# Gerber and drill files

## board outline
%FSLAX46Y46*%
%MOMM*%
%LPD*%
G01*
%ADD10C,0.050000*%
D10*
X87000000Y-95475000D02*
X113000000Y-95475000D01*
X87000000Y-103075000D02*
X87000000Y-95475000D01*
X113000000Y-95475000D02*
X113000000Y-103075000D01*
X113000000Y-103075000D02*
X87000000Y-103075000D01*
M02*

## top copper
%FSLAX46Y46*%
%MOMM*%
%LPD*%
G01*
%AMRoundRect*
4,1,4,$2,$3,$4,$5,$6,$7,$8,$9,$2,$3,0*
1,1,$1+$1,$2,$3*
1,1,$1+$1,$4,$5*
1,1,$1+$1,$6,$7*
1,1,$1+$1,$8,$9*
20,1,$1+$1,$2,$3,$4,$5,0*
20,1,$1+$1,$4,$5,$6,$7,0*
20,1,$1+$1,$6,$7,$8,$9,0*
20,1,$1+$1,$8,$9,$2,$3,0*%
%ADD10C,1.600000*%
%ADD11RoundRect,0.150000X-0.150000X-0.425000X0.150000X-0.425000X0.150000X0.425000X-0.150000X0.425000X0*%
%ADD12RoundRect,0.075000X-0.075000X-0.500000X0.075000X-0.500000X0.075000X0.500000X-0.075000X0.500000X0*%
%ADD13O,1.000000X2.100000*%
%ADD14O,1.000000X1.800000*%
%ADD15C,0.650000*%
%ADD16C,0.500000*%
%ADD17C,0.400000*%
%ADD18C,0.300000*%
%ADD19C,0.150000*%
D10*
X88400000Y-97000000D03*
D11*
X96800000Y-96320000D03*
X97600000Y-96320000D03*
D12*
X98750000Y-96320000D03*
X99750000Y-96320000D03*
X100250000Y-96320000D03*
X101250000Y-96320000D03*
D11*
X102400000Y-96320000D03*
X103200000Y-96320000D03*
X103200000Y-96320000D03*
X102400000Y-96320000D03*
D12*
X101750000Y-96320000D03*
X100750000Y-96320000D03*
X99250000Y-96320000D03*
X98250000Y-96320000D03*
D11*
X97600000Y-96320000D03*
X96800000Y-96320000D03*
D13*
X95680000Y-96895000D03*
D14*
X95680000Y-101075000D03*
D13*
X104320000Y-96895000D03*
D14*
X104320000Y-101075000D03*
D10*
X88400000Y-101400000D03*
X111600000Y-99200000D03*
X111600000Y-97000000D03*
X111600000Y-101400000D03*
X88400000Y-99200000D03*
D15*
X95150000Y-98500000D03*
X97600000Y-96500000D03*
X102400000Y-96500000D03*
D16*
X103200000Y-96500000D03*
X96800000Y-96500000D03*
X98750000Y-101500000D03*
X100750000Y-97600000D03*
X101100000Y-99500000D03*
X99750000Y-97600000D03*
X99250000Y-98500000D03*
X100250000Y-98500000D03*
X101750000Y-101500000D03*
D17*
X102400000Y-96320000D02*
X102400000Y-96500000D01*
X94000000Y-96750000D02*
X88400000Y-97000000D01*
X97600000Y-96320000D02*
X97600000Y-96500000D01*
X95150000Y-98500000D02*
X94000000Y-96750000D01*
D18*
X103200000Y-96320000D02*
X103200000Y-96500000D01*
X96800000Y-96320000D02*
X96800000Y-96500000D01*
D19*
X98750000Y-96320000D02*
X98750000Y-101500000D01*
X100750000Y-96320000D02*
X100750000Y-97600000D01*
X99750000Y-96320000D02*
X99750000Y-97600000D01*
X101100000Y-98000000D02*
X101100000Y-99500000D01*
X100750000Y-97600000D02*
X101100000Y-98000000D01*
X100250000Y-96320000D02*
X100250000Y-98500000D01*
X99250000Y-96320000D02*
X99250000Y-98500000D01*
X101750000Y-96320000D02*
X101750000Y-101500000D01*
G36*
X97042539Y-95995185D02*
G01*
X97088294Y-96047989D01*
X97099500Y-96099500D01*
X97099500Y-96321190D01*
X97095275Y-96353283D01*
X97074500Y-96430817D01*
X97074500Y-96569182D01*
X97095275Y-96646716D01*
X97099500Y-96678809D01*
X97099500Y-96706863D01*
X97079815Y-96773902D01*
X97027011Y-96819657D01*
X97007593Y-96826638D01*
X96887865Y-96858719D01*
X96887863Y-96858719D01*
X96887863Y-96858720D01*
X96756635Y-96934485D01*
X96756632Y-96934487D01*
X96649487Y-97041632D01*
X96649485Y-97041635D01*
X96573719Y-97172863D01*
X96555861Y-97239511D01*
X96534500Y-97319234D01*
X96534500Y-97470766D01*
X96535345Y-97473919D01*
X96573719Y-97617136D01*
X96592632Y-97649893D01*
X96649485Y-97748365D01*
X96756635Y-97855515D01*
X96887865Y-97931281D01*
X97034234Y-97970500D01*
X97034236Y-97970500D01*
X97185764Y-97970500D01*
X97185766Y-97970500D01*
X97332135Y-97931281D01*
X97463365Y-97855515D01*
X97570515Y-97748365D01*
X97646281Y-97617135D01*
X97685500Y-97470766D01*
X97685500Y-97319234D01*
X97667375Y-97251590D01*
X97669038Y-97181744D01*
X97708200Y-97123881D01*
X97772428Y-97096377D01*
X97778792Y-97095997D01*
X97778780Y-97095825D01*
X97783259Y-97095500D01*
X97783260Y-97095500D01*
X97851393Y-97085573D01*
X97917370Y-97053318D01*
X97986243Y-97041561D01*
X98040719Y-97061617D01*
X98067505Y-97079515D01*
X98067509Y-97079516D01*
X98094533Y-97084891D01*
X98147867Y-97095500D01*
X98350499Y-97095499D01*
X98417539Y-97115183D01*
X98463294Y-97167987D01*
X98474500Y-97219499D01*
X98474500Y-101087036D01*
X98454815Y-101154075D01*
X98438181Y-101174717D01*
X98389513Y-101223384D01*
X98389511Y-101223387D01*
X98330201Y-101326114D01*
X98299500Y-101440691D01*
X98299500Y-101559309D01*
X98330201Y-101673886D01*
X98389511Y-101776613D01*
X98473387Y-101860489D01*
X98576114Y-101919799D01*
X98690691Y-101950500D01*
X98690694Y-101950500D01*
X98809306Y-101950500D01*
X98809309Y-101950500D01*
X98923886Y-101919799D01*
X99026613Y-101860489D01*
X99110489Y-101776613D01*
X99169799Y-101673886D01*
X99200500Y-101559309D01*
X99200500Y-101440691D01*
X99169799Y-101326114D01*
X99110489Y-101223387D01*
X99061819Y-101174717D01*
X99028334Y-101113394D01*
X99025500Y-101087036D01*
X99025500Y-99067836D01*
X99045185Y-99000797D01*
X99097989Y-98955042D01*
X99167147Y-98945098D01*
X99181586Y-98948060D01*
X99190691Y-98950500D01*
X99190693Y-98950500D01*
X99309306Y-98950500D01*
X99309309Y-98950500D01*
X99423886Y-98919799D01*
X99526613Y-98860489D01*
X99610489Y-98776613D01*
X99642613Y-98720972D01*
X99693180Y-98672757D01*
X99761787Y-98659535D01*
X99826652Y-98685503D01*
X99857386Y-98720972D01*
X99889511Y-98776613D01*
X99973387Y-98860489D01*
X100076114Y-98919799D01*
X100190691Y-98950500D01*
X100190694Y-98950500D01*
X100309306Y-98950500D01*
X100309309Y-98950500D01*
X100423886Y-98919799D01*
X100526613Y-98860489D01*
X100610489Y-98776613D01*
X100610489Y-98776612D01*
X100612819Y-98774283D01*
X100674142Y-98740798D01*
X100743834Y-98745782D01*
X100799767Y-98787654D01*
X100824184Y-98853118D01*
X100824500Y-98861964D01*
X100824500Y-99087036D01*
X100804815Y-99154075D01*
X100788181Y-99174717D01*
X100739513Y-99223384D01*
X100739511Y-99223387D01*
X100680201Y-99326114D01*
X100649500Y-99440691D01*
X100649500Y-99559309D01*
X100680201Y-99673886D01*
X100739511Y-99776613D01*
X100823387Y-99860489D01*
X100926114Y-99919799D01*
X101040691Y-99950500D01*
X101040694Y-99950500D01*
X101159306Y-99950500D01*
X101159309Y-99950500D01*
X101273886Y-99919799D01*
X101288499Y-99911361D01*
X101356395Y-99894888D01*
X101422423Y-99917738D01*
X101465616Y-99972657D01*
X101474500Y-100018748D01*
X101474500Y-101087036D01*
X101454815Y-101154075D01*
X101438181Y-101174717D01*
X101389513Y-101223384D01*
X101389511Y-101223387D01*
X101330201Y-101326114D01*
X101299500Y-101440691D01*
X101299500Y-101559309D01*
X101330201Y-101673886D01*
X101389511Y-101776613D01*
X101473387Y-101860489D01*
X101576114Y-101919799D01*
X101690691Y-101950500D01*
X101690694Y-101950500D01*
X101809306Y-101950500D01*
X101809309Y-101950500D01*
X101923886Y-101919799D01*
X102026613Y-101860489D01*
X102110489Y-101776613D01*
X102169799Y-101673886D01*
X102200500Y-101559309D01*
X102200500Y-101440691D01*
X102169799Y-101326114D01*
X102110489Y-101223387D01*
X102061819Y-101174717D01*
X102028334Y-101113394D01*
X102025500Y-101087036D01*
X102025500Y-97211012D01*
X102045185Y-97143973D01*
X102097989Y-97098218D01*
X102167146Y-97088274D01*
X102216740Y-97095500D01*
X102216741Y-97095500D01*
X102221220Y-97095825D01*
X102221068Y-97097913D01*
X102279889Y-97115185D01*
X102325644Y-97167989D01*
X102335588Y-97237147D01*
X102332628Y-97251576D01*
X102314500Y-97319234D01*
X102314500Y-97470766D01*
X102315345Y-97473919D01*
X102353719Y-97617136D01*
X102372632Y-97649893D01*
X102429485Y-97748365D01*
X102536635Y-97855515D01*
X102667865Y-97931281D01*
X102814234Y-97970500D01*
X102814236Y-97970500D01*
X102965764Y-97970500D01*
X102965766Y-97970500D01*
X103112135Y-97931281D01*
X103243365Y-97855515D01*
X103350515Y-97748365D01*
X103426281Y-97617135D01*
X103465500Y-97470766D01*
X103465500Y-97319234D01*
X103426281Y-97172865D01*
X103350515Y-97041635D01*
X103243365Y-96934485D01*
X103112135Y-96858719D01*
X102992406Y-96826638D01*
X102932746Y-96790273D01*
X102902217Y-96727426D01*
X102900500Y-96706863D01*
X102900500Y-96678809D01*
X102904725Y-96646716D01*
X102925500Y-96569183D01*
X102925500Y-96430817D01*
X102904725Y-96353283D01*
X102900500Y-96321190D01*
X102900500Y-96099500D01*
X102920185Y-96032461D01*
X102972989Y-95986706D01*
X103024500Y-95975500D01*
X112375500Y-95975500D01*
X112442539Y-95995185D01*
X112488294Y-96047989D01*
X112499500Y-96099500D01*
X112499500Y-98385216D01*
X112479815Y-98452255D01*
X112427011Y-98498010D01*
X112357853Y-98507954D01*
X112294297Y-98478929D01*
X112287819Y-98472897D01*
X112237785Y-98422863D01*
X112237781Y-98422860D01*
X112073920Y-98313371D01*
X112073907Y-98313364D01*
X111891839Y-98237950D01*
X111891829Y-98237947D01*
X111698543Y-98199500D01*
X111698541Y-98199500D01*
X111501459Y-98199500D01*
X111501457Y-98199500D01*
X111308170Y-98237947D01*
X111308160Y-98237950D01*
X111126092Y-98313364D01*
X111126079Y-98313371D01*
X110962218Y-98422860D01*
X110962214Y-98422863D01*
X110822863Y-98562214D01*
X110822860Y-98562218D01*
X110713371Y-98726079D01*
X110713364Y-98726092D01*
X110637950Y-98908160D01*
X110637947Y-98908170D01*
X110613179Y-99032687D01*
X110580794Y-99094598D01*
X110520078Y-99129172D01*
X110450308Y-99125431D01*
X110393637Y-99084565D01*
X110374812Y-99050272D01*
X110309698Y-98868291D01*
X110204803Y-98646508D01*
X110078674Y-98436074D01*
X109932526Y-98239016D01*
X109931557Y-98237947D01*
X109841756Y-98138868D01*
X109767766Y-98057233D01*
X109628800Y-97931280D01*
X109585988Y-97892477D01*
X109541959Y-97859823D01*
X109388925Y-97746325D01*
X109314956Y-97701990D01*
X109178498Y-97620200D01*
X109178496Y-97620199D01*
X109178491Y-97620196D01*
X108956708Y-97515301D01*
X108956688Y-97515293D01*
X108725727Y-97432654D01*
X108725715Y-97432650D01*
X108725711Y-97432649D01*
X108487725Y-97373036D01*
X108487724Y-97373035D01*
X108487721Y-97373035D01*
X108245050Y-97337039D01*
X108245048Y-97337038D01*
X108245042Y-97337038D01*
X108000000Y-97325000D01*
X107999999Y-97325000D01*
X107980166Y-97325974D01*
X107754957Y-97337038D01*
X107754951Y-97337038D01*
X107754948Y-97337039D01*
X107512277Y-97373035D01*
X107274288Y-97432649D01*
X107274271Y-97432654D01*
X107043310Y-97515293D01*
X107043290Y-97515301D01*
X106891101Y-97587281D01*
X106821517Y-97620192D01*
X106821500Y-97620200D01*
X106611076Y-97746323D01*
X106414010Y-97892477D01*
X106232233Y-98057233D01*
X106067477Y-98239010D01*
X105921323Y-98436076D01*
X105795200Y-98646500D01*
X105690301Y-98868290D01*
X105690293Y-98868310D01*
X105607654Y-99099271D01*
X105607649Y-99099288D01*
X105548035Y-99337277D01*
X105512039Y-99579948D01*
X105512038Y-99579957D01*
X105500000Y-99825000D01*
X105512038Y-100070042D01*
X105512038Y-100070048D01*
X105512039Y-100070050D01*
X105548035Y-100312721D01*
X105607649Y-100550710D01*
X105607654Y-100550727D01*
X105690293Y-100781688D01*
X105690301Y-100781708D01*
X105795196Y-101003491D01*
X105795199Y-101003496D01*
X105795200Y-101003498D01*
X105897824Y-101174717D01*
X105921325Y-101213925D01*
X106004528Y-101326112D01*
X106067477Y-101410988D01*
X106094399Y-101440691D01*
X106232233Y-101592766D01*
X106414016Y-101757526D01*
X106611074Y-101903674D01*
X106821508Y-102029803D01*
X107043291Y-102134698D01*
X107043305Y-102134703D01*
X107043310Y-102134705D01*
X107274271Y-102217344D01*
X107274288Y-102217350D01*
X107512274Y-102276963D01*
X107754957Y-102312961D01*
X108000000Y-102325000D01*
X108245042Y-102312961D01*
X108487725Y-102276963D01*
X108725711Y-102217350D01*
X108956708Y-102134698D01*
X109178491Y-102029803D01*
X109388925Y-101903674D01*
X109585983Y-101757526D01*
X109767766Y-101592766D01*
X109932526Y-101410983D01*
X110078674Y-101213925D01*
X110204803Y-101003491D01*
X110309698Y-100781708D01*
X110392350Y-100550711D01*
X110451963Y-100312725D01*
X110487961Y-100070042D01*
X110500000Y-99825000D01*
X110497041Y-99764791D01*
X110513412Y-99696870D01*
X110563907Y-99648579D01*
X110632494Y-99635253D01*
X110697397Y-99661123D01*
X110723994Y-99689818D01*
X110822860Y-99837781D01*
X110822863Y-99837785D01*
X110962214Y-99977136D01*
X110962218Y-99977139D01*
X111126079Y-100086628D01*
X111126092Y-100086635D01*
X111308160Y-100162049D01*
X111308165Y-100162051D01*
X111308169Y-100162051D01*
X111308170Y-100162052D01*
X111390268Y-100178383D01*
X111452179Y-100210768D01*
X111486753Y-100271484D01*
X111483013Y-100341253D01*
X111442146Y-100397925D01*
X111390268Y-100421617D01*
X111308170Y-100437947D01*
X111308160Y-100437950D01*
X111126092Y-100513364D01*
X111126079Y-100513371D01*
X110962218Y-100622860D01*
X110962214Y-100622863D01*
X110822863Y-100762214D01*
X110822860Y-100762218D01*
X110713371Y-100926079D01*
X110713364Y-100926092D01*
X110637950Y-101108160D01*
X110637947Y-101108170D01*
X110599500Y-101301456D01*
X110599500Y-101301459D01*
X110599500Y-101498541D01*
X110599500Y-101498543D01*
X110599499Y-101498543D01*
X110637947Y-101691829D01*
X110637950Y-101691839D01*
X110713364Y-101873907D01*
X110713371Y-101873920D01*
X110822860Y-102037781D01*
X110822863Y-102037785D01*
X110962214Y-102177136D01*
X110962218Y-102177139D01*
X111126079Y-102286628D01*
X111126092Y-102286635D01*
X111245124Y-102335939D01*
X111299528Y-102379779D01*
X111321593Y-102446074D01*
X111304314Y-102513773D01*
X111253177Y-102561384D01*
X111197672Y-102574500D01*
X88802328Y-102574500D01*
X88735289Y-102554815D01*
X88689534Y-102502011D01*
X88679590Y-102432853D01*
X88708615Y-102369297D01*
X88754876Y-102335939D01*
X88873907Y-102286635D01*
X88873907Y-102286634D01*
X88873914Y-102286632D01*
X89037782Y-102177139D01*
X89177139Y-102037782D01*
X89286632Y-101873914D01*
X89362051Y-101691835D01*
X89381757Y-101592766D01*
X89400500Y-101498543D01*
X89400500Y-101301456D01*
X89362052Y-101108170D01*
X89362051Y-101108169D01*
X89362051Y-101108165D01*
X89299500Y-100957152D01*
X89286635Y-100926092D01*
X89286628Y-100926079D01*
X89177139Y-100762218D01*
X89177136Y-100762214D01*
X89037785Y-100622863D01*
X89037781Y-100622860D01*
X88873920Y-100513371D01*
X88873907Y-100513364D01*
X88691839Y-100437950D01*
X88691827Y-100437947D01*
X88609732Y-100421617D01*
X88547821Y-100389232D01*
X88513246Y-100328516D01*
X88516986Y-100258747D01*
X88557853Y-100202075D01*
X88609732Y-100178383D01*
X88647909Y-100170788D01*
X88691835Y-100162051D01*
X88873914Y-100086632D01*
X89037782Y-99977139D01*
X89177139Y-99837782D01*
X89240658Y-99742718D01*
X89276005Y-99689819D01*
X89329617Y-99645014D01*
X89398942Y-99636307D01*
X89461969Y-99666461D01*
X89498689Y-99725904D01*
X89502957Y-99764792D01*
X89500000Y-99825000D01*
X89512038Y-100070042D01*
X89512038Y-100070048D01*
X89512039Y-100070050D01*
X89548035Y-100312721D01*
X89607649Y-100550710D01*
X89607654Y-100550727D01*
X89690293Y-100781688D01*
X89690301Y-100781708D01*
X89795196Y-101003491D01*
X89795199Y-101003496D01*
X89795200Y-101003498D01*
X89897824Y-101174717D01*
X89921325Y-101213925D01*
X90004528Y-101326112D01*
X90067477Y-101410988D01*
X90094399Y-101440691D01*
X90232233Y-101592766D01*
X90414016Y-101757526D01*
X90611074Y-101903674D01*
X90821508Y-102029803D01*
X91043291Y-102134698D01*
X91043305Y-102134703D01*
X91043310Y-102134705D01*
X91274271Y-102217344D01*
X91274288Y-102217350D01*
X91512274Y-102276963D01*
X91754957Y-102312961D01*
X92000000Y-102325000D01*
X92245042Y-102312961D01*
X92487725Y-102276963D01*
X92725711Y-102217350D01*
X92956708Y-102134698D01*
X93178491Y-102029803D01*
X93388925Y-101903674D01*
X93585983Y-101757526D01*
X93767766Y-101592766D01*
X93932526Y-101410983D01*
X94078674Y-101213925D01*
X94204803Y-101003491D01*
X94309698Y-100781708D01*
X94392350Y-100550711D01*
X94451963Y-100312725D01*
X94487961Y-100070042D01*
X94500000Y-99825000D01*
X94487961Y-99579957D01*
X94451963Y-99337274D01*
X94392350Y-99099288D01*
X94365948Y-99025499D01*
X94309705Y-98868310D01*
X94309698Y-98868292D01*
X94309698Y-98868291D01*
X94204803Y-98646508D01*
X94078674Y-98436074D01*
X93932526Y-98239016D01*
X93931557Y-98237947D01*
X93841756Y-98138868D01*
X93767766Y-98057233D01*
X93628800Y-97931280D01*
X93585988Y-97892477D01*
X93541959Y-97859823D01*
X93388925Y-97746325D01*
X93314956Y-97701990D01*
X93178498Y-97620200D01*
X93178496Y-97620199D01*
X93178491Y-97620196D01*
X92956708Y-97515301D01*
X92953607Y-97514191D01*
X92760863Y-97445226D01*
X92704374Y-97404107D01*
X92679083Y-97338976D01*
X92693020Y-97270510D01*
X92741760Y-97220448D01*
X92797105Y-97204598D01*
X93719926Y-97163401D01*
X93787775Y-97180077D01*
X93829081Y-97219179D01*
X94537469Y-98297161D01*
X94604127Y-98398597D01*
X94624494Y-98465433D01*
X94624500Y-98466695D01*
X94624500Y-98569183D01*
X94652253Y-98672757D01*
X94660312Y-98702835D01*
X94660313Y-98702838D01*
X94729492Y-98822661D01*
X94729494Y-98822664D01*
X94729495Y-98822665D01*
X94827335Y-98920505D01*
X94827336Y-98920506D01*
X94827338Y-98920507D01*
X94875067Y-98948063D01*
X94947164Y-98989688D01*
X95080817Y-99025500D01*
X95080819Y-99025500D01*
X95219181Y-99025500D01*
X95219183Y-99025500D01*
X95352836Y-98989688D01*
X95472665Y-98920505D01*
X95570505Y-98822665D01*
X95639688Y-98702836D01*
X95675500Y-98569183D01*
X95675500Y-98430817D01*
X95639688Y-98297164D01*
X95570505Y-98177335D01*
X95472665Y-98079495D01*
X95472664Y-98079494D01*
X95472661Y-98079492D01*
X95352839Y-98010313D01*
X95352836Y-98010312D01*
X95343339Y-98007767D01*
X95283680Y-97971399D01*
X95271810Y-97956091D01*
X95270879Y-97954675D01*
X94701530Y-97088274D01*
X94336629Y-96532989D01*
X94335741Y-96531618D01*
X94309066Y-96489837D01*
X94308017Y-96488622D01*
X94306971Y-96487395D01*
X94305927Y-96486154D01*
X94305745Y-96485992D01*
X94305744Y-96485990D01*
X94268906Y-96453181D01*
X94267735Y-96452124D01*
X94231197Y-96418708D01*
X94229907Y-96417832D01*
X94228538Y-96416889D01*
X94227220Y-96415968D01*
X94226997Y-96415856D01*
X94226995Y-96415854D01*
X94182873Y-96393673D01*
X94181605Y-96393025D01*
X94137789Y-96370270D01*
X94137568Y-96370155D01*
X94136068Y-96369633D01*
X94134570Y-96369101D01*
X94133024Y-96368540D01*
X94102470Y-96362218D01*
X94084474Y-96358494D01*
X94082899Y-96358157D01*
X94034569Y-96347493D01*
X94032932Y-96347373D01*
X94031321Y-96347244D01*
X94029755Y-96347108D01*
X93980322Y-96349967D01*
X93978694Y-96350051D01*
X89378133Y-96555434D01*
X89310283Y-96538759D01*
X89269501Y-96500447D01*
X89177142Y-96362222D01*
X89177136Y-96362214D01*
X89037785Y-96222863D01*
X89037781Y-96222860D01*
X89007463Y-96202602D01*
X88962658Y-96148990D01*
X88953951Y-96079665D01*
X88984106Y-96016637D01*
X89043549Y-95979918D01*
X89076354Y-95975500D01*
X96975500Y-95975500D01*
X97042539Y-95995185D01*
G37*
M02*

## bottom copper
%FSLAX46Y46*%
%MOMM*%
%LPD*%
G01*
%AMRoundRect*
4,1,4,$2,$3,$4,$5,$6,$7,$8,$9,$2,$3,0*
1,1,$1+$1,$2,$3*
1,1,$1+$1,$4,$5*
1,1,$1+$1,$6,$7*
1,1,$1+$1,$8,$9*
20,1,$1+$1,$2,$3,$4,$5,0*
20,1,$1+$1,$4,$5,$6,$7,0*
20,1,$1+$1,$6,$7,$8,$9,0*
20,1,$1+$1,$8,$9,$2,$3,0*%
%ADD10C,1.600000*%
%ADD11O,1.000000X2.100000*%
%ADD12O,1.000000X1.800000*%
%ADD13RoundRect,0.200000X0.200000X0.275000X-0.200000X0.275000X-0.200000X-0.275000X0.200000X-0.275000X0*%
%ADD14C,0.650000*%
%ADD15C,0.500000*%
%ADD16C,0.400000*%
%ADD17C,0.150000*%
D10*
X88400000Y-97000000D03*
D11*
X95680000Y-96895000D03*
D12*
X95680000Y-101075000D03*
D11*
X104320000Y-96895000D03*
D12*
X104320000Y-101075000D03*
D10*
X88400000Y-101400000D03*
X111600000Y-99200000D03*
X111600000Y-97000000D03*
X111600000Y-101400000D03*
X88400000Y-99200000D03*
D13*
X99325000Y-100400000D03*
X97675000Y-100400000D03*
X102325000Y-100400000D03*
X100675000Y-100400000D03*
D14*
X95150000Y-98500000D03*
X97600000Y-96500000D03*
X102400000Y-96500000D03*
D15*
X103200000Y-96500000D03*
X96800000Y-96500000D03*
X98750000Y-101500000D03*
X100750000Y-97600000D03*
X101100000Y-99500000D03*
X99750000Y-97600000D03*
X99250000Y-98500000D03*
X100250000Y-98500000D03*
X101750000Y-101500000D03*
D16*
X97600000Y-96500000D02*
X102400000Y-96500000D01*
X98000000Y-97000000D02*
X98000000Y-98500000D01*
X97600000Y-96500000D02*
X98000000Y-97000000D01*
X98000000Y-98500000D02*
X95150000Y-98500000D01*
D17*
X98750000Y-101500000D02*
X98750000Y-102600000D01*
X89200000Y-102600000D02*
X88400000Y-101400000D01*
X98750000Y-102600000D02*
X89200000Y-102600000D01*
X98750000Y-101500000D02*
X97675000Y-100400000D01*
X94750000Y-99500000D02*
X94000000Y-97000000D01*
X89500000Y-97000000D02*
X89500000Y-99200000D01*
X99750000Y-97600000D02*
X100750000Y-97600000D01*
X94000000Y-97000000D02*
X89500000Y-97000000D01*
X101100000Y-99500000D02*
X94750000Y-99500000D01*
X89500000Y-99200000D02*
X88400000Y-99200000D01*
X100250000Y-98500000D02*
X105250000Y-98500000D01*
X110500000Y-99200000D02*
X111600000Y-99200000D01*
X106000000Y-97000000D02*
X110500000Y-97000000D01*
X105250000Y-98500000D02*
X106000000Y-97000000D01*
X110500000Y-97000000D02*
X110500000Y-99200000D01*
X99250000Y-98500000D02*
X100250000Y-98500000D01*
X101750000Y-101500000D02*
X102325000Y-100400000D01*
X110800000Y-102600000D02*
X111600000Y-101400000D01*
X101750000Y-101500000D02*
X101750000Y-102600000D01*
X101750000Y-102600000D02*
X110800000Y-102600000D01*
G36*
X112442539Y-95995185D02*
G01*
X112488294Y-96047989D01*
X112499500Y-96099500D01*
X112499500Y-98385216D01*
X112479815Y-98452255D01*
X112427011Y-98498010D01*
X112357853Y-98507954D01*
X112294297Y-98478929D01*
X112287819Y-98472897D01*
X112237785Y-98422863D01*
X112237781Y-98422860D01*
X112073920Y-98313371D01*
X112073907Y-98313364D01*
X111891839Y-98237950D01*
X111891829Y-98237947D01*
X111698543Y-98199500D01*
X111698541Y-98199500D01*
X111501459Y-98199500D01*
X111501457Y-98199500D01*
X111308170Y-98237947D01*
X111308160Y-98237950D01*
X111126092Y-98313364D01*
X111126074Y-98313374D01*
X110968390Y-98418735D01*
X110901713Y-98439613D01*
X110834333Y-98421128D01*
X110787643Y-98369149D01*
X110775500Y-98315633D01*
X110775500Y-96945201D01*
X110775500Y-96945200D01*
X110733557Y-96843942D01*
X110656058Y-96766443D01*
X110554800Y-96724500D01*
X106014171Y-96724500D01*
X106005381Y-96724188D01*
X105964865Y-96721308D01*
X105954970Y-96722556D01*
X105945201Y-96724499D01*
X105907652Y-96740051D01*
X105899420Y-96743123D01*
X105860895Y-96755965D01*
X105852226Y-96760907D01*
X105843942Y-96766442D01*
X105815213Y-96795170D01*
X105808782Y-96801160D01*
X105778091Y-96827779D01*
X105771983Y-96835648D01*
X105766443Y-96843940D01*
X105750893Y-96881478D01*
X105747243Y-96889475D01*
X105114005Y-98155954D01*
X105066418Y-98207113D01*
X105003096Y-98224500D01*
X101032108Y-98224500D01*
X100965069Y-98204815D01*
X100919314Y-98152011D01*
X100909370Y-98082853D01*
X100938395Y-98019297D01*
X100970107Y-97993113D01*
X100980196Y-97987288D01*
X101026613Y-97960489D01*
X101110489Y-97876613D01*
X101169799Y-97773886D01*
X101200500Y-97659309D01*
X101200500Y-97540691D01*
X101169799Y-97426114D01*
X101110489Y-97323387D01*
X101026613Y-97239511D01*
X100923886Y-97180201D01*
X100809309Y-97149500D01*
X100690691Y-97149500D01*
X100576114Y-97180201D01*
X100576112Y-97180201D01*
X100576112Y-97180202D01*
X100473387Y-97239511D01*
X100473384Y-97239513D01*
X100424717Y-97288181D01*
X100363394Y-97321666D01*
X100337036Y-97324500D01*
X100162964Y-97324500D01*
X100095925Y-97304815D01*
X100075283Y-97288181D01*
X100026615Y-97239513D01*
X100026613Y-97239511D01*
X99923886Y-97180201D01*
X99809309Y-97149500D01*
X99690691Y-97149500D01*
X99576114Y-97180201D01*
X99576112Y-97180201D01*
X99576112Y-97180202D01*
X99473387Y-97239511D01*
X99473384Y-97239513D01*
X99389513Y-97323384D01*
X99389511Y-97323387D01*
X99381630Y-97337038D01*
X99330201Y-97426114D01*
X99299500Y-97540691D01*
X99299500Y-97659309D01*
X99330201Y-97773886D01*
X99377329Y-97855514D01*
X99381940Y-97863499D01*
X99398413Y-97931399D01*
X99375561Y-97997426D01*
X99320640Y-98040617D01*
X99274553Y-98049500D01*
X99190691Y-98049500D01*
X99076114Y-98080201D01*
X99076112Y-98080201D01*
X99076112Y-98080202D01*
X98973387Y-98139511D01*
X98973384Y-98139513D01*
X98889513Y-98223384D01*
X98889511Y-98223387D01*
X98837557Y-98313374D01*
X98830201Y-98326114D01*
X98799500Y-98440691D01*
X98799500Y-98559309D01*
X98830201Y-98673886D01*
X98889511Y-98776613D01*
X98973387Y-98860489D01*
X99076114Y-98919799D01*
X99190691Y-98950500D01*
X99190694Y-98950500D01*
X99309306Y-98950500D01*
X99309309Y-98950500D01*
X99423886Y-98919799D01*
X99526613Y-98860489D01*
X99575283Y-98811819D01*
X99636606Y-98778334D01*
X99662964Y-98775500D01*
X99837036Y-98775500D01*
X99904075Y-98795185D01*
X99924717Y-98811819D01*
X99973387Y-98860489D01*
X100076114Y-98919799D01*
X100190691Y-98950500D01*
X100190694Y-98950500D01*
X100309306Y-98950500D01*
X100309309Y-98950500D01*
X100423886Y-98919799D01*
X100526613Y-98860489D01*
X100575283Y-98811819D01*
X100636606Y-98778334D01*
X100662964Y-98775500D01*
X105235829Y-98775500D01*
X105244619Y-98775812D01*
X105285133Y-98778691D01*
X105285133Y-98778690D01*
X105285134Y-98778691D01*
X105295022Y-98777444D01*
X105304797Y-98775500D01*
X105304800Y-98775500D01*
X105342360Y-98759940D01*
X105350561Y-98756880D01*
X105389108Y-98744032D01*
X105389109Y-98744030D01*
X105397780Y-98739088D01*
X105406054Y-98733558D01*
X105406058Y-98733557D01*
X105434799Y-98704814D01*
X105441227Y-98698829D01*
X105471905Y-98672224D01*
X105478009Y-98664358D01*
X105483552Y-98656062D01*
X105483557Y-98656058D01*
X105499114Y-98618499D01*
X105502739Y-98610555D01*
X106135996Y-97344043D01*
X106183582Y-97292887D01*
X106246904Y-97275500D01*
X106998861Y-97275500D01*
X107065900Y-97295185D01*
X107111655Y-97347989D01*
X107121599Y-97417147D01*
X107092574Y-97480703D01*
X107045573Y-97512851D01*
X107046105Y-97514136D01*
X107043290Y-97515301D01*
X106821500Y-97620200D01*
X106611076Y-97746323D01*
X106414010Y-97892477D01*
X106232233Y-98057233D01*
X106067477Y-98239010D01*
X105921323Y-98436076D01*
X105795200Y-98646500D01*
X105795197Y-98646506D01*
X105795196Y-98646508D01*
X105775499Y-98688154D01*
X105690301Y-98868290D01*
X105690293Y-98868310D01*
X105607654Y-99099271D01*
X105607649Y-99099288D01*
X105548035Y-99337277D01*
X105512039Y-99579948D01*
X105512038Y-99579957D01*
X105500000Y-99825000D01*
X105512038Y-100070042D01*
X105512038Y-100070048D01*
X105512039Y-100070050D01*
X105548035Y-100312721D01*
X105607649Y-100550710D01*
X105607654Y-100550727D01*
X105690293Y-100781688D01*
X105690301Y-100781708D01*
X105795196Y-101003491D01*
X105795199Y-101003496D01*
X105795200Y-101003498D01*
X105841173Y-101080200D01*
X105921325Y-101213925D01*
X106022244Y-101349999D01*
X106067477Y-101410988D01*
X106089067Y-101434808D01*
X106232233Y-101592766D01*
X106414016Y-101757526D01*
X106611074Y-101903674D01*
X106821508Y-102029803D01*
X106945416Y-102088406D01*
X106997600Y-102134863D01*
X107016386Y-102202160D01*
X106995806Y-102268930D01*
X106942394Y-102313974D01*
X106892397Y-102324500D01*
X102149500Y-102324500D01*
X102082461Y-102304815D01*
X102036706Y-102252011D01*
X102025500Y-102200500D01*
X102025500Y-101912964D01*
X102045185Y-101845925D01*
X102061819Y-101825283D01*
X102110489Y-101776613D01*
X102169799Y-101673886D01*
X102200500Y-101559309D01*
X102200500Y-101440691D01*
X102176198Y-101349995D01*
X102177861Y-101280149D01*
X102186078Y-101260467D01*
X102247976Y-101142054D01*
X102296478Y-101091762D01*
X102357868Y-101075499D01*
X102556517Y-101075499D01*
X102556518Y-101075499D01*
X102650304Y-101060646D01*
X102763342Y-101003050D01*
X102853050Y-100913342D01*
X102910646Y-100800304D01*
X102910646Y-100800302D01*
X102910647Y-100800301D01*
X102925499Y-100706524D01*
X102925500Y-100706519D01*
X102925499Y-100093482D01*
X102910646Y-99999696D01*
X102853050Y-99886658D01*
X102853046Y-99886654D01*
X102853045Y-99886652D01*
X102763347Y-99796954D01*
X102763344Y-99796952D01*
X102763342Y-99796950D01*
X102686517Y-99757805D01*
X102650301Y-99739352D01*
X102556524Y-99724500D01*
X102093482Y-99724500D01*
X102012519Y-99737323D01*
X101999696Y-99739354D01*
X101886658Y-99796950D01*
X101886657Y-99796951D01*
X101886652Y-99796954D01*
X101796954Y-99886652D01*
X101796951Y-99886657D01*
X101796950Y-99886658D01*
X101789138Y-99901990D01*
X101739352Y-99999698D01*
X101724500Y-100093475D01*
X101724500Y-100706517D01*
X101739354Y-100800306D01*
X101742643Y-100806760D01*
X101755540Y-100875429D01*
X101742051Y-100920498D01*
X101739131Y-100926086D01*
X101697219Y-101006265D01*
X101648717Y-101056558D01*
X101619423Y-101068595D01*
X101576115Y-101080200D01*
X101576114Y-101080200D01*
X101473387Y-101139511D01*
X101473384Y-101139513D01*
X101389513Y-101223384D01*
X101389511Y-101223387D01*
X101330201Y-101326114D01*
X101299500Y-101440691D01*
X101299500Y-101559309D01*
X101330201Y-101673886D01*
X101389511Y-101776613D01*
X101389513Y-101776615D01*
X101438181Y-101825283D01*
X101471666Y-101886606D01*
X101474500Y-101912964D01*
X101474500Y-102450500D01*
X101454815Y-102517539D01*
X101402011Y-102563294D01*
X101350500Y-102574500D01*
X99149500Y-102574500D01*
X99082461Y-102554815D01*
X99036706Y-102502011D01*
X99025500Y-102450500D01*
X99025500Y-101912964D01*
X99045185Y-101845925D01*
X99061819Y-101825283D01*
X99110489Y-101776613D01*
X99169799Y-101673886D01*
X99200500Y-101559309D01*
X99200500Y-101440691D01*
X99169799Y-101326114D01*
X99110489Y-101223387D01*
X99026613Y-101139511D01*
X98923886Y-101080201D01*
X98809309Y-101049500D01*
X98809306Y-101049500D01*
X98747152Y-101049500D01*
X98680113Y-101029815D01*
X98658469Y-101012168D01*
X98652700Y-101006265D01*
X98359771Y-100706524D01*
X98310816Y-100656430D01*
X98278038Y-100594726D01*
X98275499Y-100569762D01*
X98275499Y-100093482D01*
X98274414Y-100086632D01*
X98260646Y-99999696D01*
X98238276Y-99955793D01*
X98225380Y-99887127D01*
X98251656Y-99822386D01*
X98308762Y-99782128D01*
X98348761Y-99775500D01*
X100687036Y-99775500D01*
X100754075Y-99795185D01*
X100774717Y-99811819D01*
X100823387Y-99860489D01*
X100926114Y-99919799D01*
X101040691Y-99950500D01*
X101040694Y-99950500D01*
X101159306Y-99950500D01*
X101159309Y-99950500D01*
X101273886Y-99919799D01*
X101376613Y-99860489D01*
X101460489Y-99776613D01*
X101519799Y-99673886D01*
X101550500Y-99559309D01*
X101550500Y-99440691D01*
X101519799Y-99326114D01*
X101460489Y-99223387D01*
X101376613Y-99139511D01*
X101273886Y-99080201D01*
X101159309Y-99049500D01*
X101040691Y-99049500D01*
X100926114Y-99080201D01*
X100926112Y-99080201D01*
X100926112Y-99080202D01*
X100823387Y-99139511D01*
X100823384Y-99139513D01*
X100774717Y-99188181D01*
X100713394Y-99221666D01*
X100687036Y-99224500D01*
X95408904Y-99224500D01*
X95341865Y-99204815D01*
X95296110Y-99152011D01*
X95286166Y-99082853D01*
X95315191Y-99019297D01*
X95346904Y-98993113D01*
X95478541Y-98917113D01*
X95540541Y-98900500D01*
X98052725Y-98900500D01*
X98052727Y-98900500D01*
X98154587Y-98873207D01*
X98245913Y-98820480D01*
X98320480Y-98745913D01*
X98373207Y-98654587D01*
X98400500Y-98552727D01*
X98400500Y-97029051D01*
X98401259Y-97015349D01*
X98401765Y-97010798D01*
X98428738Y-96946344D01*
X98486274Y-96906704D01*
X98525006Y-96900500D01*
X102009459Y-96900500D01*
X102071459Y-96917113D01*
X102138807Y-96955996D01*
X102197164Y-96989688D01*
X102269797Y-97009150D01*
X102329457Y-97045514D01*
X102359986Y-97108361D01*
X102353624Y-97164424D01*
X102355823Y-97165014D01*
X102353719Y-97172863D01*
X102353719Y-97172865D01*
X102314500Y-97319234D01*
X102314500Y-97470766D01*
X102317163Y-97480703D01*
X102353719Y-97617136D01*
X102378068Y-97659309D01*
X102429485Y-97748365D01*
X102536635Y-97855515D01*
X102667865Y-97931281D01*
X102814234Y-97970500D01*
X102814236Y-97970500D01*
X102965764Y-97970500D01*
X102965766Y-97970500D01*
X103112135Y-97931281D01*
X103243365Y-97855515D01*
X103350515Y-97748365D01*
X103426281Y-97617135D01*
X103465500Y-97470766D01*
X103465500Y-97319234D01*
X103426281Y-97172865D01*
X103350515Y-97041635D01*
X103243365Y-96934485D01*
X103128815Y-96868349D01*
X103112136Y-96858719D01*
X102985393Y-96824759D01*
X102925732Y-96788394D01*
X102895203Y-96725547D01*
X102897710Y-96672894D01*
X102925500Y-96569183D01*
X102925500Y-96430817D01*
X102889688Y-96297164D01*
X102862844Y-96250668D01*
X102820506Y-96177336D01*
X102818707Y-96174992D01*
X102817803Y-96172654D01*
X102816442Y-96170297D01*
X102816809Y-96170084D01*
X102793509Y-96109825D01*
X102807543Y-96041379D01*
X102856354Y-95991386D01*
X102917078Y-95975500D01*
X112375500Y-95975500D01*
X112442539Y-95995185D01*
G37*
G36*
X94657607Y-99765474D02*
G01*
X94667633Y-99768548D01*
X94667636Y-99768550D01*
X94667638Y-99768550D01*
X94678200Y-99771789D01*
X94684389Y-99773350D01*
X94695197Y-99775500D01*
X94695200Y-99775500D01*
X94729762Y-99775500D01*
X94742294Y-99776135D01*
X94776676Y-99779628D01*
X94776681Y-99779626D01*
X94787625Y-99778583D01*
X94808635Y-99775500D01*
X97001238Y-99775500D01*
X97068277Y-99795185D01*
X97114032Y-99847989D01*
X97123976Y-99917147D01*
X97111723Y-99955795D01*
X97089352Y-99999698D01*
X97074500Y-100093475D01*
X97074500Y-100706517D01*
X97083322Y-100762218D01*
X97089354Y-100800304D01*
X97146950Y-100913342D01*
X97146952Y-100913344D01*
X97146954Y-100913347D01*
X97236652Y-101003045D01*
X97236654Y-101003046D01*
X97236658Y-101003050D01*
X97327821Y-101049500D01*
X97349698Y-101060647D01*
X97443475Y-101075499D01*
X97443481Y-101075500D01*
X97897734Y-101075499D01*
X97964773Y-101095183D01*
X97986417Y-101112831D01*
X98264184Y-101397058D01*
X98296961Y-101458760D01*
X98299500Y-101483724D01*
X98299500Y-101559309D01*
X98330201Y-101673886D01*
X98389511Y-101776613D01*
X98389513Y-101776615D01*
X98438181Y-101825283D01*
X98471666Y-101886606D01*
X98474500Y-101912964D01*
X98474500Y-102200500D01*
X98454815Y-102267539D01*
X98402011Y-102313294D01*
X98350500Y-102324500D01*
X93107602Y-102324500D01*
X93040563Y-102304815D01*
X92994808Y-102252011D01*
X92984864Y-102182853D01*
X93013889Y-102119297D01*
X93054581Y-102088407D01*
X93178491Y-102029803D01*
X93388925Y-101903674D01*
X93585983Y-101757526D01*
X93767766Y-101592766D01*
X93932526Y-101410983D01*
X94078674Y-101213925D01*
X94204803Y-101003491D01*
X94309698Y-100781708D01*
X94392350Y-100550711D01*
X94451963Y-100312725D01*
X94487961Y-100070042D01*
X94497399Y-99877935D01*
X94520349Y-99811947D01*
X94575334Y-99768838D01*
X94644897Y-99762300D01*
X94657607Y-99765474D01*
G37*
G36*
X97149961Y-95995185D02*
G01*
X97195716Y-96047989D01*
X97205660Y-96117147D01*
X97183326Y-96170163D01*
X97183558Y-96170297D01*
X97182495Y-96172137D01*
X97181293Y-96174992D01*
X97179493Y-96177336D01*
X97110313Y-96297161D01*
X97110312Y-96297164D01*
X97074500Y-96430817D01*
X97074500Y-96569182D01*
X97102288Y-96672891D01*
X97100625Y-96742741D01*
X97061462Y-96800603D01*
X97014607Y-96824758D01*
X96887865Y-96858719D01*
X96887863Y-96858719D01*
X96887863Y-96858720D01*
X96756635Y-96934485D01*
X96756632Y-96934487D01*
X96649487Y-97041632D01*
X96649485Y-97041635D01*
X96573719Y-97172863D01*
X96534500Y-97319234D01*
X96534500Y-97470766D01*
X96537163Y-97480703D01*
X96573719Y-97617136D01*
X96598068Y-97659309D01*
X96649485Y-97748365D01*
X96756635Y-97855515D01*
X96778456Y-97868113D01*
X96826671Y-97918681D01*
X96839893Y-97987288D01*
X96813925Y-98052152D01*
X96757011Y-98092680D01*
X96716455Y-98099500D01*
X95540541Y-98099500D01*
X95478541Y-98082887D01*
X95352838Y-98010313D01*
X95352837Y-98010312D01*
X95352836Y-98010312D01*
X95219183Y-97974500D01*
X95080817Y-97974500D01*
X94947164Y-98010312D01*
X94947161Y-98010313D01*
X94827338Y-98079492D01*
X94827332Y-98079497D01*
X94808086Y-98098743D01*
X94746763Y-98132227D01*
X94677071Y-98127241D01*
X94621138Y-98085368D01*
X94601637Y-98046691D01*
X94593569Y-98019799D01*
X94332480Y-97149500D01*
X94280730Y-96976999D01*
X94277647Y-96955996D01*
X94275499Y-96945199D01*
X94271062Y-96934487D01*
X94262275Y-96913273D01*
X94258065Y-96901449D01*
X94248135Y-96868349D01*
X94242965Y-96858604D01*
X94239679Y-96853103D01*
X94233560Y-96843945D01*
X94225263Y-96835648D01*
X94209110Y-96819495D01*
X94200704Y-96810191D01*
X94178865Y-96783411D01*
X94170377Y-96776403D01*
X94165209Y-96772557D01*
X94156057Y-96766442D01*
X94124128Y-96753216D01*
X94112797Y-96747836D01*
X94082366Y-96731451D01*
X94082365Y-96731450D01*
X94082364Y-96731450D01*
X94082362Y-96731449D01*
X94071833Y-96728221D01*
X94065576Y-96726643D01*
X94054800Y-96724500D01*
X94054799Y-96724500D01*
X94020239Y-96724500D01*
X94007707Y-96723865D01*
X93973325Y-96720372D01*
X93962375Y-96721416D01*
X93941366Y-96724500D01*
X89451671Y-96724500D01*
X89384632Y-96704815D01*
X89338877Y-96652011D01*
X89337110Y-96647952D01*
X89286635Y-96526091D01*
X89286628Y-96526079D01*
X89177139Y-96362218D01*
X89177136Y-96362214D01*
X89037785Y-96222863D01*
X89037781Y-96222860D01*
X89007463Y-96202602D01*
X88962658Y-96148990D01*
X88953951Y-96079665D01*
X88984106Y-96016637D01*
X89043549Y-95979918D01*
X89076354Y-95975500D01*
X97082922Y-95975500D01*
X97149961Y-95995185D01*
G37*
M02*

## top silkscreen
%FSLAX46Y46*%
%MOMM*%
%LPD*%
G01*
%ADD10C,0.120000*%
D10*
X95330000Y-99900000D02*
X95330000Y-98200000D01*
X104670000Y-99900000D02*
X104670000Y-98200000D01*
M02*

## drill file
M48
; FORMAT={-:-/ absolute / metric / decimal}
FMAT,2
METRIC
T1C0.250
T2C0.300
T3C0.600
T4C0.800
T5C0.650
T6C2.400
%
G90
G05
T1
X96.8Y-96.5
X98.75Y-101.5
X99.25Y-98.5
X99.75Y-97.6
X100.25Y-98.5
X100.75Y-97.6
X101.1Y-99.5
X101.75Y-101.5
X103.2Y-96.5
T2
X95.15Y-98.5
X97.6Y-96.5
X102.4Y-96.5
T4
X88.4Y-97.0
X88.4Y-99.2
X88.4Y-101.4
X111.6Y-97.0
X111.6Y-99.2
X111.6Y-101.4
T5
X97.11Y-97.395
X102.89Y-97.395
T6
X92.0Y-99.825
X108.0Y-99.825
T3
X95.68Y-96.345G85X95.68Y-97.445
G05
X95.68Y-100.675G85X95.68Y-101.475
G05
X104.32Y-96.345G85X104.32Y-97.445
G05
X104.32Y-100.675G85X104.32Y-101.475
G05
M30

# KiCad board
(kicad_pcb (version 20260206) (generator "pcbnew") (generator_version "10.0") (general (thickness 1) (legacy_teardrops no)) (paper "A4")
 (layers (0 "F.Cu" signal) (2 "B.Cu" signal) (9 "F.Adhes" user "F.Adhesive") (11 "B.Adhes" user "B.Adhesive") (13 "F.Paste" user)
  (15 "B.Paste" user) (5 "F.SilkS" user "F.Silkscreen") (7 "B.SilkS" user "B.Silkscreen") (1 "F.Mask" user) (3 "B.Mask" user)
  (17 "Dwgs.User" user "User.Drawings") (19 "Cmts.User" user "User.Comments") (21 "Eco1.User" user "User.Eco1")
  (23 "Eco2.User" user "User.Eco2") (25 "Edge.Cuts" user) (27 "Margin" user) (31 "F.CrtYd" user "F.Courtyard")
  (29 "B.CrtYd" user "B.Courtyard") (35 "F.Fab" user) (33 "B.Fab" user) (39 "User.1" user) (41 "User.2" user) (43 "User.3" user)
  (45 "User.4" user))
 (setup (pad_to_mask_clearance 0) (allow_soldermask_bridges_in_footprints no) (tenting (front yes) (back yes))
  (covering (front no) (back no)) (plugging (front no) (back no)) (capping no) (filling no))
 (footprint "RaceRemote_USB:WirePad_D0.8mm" (layer "F.Cu") (at 88.4 97)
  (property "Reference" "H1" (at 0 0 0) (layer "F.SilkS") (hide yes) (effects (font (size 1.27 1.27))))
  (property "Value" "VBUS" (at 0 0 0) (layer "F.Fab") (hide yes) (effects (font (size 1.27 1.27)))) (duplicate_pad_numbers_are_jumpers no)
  (pad "1" thru_hole circle (at 0 0) (size 1.6 1.6) (drill 0.8) (layers "*.Cu" "*.Mask") (remove_unused_layers no) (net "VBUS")))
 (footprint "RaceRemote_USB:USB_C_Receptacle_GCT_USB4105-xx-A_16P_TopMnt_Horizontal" (layer "F.Cu") (at 100 100)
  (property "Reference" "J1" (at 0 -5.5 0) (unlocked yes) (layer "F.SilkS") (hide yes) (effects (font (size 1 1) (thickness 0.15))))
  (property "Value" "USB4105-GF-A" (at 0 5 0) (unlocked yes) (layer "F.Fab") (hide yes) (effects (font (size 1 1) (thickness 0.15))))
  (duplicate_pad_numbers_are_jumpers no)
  (fp_line (start -4.67 -0.1) (end -4.67 -1.8) (stroke (width 0.12) (type solid)) (layer "F.SilkS"))
  (fp_line (start 4.67 -0.1) (end 4.67 -1.8) (stroke (width 0.12) (type solid)) (layer "F.SilkS"))
  (pad "" np_thru_hole circle (at -2.89 -2.605) (size 0.65 0.65) (drill 0.65) (layers "*.Cu" "*.Mask"))
  (pad "" np_thru_hole circle (at 2.89 -2.605) (size 0.65 0.65) (drill 0.65) (layers "*.Cu" "*.Mask"))
  (pad "A1" smd roundrect (at -3.2 -3.68) (size 0.6 1.15) (layers "F.Cu" "F.Mask" "F.Paste") (roundrect_rratio 0.25) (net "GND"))
  (pad "A4" smd roundrect (at -2.4 -3.68) (size 0.6 1.15) (layers "F.Cu" "F.Mask" "F.Paste") (roundrect_rratio 0.25) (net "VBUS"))
  (pad "A5" smd roundrect (at -1.25 -3.68) (size 0.3 1.15) (layers "F.Cu" "F.Mask" "F.Paste") (roundrect_rratio 0.25) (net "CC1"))
  (pad "A6" smd roundrect (at -0.25 -3.68) (size 0.3 1.15) (layers "F.Cu" "F.Mask" "F.Paste") (roundrect_rratio 0.25) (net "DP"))
  (pad "A7" smd roundrect (at 0.25 -3.68) (size 0.3 1.15) (layers "F.Cu" "F.Mask" "F.Paste") (roundrect_rratio 0.25) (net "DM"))
  (pad "A8" smd roundrect (at 1.25 -3.68) (size 0.3 1.15) (layers "F.Cu" "F.Mask" "F.Paste") (roundrect_rratio 0.25)
   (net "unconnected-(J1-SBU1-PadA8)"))
  (pad "A9" smd roundrect (at 2.4 -3.68) (size 0.6 1.15) (layers "F.Cu" "F.Mask" "F.Paste") (roundrect_rratio 0.25) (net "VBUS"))
  (pad "A12" smd roundrect (at 3.2 -3.68) (size 0.6 1.15) (layers "F.Cu" "F.Mask" "F.Paste") (roundrect_rratio 0.25) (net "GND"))
  (pad "B1" smd roundrect (at 3.2 -3.68) (size 0.6 1.15) (layers "F.Cu" "F.Mask" "F.Paste") (roundrect_rratio 0.25) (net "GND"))
  (pad "B4" smd roundrect (at 2.4 -3.68) (size 0.6 1.15) (layers "F.Cu" "F.Mask" "F.Paste") (roundrect_rratio 0.25) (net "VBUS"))
  (pad "B5" smd roundrect (at 1.75 -3.68) (size 0.3 1.15) (layers "F.Cu" "F.Mask" "F.Paste") (roundrect_rratio 0.25) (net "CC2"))
  (pad "B6" smd roundrect (at 0.75 -3.68) (size 0.3 1.15) (layers "F.Cu" "F.Mask" "F.Paste") (roundrect_rratio 0.25) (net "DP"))
  (pad "B7" smd roundrect (at -0.75 -3.68) (size 0.3 1.15) (layers "F.Cu" "F.Mask" "F.Paste") (roundrect_rratio 0.25) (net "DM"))
  (pad "B8" smd roundrect (at -1.75 -3.68) (size 0.3 1.15) (layers "F.Cu" "F.Mask" "F.Paste") (roundrect_rratio 0.25)
   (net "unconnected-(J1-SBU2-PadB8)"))
  (pad "B9" smd roundrect (at -2.4 -3.68) (size 0.6 1.15) (layers "F.Cu" "F.Mask" "F.Paste") (roundrect_rratio 0.25) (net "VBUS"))
  (pad "B12" smd roundrect (at -3.2 -3.68) (size 0.6 1.15) (layers "F.Cu" "F.Mask" "F.Paste") (roundrect_rratio 0.25) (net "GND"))
  (pad "S1" thru_hole oval (at -4.32 -3.105) (size 1 2.1) (drill oval 0.6 1.7) (layers "*.Cu" "*.Mask" "F.Paste") (remove_unused_layers no)
   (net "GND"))
  (pad "S1" thru_hole oval (at -4.32 1.075) (size 1 1.8) (drill oval 0.6 1.4) (layers "*.Cu" "*.Mask" "F.Paste") (remove_unused_layers no)
   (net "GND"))
  (pad "S1" thru_hole oval (at 4.32 -3.105) (size 1 2.1) (drill oval 0.6 1.7) (layers "*.Cu" "*.Mask" "F.Paste") (remove_unused_layers no)
   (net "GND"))
  (pad "S1" thru_hole oval (at 4.32 1.075) (size 1 1.8) (drill oval 0.6 1.4) (layers "*.Cu" "*.Mask" "F.Paste") (remove_unused_layers no)
   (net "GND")))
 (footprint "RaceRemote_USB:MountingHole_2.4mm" (layer "F.Cu") (at 92 99.825)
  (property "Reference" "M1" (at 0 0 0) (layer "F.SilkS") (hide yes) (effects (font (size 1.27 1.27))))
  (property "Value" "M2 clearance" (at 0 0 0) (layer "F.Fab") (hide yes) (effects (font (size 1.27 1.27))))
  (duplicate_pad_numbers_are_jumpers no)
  (pad "" np_thru_hole circle (at 0 0) (size 2.4 2.4) (drill 2.4) (layers "*.Cu" "*.Mask")))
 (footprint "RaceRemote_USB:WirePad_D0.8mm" (layer "F.Cu") (at 88.4 101.4)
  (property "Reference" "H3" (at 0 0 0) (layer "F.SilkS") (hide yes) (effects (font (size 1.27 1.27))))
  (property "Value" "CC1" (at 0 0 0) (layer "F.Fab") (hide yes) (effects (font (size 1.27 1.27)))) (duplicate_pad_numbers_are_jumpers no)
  (pad "1" thru_hole circle (at 0 0) (size 1.6 1.6) (drill 0.8) (layers "*.Cu" "*.Mask") (remove_unused_layers no) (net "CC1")))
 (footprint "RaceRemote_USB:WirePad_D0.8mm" (layer "F.Cu") (at 111.6 99.2)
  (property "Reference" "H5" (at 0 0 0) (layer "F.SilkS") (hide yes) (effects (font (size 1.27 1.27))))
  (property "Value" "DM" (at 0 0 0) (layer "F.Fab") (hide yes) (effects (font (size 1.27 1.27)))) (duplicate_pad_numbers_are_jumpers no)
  (pad "1" thru_hole circle (at 0 0) (size 1.6 1.6) (drill 0.8) (layers "*.Cu" "*.Mask") (remove_unused_layers no) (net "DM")))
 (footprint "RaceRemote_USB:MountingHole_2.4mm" (layer "F.Cu") (at 108 99.825)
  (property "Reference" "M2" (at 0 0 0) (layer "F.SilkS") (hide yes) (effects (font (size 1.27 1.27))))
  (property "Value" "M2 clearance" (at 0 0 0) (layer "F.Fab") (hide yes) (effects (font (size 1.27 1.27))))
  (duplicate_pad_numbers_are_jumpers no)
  (pad "" np_thru_hole circle (at 0 0) (size 2.4 2.4) (drill 2.4) (layers "*.Cu" "*.Mask")))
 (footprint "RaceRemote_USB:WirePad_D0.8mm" (layer "F.Cu") (at 111.6 97)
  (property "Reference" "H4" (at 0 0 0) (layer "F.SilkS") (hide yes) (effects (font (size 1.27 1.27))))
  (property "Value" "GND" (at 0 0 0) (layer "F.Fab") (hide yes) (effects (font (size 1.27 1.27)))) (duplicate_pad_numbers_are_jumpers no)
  (pad "1" thru_hole circle (at 0 0) (size 1.6 1.6) (drill 0.8) (layers "*.Cu" "*.Mask") (remove_unused_layers no) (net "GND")))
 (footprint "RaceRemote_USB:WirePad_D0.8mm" (layer "F.Cu") (at 111.6 101.4)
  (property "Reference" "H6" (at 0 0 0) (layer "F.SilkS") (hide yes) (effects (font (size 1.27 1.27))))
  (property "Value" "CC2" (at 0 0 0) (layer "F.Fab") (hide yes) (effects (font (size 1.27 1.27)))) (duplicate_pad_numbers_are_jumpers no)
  (pad "1" thru_hole circle (at 0 0) (size 1.6 1.6) (drill 0.8) (layers "*.Cu" "*.Mask") (remove_unused_layers no) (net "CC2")))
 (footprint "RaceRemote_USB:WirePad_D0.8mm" (layer "F.Cu") (at 88.4 99.2)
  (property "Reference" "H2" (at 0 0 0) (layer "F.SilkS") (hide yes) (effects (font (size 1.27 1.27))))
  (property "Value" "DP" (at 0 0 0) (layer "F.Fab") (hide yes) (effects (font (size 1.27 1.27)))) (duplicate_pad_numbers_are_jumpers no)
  (pad "1" thru_hole circle (at 0 0) (size 1.6 1.6) (drill 0.8) (layers "*.Cu" "*.Mask") (remove_unused_layers no) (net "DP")))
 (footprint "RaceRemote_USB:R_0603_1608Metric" (layer "B.Cu") (at 98.5 100.4 180)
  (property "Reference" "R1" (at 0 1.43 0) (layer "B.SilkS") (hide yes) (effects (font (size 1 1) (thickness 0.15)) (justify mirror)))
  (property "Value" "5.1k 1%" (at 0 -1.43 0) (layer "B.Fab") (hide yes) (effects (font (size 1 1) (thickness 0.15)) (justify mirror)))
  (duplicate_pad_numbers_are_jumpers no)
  (pad "1" smd roundrect (at -0.825 0 180) (size 0.8 0.95) (layers "B.Cu" "B.Mask" "B.Paste") (roundrect_rratio 0.25) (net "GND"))
  (pad "2" smd roundrect (at 0.825 0 180) (size 0.8 0.95) (layers "B.Cu" "B.Mask" "B.Paste") (roundrect_rratio 0.25) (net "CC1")))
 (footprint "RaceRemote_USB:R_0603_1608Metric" (layer "B.Cu") (at 101.5 100.4 180)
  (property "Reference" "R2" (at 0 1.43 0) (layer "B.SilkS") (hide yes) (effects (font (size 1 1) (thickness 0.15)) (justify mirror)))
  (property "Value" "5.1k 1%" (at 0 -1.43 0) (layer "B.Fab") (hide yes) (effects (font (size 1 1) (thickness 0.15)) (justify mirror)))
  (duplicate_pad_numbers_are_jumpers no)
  (pad "1" smd roundrect (at -0.825 0 180) (size 0.8 0.95) (layers "B.Cu" "B.Mask" "B.Paste") (roundrect_rratio 0.25) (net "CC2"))
  (pad "2" smd roundrect (at 0.825 0 180) (size 0.8 0.95) (layers "B.Cu" "B.Mask" "B.Paste") (roundrect_rratio 0.25) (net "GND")))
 (gr_line (start 87 95.475) (end 113 95.475) (stroke (width 0.05) (type default)) (layer "Edge.Cuts"))
 (gr_line (start 87 103.075) (end 87 95.475) (stroke (width 0.05) (type default)) (layer "Edge.Cuts"))
 (gr_line (start 113 95.475) (end 113 103.075) (stroke (width 0.05) (type default)) (layer "Edge.Cuts"))
 (gr_line (start 113 103.075) (end 87 103.075) (stroke (width 0.05) (type default)) (layer "Edge.Cuts"))
 (segment (start 102.4 96.32) (end 102.4 96.5) (width 0.4) (layer "F.Cu") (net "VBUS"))
 (segment (start 94 96.75) (end 88.4 97) (width 0.4) (layer "F.Cu") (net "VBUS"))
 (segment (start 97.6 96.32) (end 97.6 96.5) (width 0.4) (layer "F.Cu") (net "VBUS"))
 (segment (start 95.15 98.5) (end 94 96.75) (width 0.4) (layer "F.Cu") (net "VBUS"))
 (via (at 95.15 98.5) (size 0.65) (drill 0.3) (layers "F.Cu" "B.Cu") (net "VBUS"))
 (via (at 97.6 96.5) (size 0.65) (drill 0.3) (layers "F.Cu" "B.Cu") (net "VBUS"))
 (via (at 102.4 96.5) (size 0.65) (drill 0.3) (layers "F.Cu" "B.Cu") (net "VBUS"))
 (segment (start 97.6 96.5) (end 102.4 96.5) (width 0.4) (layer "B.Cu") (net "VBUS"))
 (segment (start 98 97) (end 98 98.5) (width 0.4) (layer "B.Cu") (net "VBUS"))
 (segment (start 97.6 96.5) (end 98 97) (width 0.4) (layer "B.Cu") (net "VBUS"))
 (segment (start 98 98.5) (end 95.15 98.5) (width 0.4) (layer "B.Cu") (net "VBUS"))
 (segment (start 103.2 96.32) (end 103.2 96.5) (width 0.3) (layer "F.Cu") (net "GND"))
 (segment (start 96.8 96.32) (end 96.8 96.5) (width 0.3) (layer "F.Cu") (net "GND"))
 (via (at 103.2 96.5) (size 0.5) (drill 0.25) (layers "F.Cu" "B.Cu") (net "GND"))
 (via (at 96.8 96.5) (size 0.5) (drill 0.25) (layers "F.Cu" "B.Cu") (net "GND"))
 (segment (start 98.75 96.32) (end 98.75 101.5) (width 0.15) (layer "F.Cu") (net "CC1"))
 (via (at 98.75 101.5) (size 0.5) (drill 0.25) (layers "F.Cu" "B.Cu") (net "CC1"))
 (segment (start 98.75 101.5) (end 98.75 102.6) (width 0.15) (layer "B.Cu") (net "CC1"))
 (segment (start 89.2 102.6) (end 88.4 101.4) (width 0.15) (layer "B.Cu") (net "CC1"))
 (segment (start 98.75 102.6) (end 89.2 102.6) (width 0.15) (layer "B.Cu") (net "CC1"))
 (segment (start 98.75 101.5) (end 97.675 100.4) (width 0.15) (layer "B.Cu") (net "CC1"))
 (segment (start 100.75 96.32) (end 100.75 97.6) (width 0.15) (layer "F.Cu") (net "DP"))
 (segment (start 99.75 96.32) (end 99.75 97.6) (width 0.15) (layer "F.Cu") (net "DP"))
 (segment (start 101.1 98) (end 101.1 99.5) (width 0.15) (layer "F.Cu") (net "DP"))
 (segment (start 100.75 97.6) (end 101.1 98) (width 0.15) (layer "F.Cu") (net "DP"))
 (via (at 100.75 97.6) (size 0.5) (drill 0.25) (layers "F.Cu" "B.Cu") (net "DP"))
 (via (at 101.1 99.5) (size 0.5) (drill 0.25) (layers "F.Cu" "B.Cu") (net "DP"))
 (via (at 99.75 97.6) (size 0.5) (drill 0.25) (layers "F.Cu" "B.Cu") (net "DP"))
 (segment (start 94.75 99.5) (end 94 97) (width 0.15) (layer "B.Cu") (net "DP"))
 (segment (start 89.5 97) (end 89.5 99.2) (width 0.15) (layer "B.Cu") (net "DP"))
 (segment (start 99.75 97.6) (end 100.75 97.6) (width 0.15) (layer "B.Cu") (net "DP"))
 (segment (start 94 97) (end 89.5 97) (width 0.15) (layer "B.Cu") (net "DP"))
 (segment (start 101.1 99.5) (end 94.75 99.5) (width 0.15) (layer "B.Cu") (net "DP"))
 (segment (start 89.5 99.2) (end 88.4 99.2) (width 0.15) (layer "B.Cu") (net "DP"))
 (segment (start 100.25 96.32) (end 100.25 98.5) (width 0.15) (layer "F.Cu") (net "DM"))
 (segment (start 99.25 96.32) (end 99.25 98.5) (width 0.15) (layer "F.Cu") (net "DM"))
 (via (at 99.25 98.5) (size 0.5) (drill 0.25) (layers "F.Cu" "B.Cu") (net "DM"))
 (via (at 100.25 98.5) (size 0.5) (drill 0.25) (layers "F.Cu" "B.Cu") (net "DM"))
 (segment (start 100.25 98.5) (end 105.25 98.5) (width 0.15) (layer "B.Cu") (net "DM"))
 (segment (start 110.5 99.2) (end 111.6 99.2) (width 0.15) (layer "B.Cu") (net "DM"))
 (segment (start 106 97) (end 110.5 97) (width 0.15) (layer "B.Cu") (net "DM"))
 (segment (start 105.25 98.5) (end 106 97) (width 0.15) (layer "B.Cu") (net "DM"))
 (segment (start 110.5 97) (end 110.5 99.2) (width 0.15) (layer "B.Cu") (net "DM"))
 (segment (start 99.25 98.5) (end 100.25 98.5) (width 0.15) (layer "B.Cu") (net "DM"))
 (segment (start 101.75 96.32) (end 101.75 101.5) (width 0.15) (layer "F.Cu") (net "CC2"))
 (via (at 101.75 101.5) (size 0.5) (drill 0.25) (layers "F.Cu" "B.Cu") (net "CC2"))
 (segment (start 101.75 101.5) (end 102.325 100.4) (width 0.15) (layer "B.Cu") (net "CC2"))
 (segment (start 110.8 102.6) (end 111.6 101.4) (width 0.15) (layer "B.Cu") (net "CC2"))
 (segment (start 101.75 101.5) (end 101.75 102.6) (width 0.15) (layer "B.Cu") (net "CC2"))
 (segment (start 101.75 102.6) (end 110.8 102.6) (width 0.15) (layer "B.Cu") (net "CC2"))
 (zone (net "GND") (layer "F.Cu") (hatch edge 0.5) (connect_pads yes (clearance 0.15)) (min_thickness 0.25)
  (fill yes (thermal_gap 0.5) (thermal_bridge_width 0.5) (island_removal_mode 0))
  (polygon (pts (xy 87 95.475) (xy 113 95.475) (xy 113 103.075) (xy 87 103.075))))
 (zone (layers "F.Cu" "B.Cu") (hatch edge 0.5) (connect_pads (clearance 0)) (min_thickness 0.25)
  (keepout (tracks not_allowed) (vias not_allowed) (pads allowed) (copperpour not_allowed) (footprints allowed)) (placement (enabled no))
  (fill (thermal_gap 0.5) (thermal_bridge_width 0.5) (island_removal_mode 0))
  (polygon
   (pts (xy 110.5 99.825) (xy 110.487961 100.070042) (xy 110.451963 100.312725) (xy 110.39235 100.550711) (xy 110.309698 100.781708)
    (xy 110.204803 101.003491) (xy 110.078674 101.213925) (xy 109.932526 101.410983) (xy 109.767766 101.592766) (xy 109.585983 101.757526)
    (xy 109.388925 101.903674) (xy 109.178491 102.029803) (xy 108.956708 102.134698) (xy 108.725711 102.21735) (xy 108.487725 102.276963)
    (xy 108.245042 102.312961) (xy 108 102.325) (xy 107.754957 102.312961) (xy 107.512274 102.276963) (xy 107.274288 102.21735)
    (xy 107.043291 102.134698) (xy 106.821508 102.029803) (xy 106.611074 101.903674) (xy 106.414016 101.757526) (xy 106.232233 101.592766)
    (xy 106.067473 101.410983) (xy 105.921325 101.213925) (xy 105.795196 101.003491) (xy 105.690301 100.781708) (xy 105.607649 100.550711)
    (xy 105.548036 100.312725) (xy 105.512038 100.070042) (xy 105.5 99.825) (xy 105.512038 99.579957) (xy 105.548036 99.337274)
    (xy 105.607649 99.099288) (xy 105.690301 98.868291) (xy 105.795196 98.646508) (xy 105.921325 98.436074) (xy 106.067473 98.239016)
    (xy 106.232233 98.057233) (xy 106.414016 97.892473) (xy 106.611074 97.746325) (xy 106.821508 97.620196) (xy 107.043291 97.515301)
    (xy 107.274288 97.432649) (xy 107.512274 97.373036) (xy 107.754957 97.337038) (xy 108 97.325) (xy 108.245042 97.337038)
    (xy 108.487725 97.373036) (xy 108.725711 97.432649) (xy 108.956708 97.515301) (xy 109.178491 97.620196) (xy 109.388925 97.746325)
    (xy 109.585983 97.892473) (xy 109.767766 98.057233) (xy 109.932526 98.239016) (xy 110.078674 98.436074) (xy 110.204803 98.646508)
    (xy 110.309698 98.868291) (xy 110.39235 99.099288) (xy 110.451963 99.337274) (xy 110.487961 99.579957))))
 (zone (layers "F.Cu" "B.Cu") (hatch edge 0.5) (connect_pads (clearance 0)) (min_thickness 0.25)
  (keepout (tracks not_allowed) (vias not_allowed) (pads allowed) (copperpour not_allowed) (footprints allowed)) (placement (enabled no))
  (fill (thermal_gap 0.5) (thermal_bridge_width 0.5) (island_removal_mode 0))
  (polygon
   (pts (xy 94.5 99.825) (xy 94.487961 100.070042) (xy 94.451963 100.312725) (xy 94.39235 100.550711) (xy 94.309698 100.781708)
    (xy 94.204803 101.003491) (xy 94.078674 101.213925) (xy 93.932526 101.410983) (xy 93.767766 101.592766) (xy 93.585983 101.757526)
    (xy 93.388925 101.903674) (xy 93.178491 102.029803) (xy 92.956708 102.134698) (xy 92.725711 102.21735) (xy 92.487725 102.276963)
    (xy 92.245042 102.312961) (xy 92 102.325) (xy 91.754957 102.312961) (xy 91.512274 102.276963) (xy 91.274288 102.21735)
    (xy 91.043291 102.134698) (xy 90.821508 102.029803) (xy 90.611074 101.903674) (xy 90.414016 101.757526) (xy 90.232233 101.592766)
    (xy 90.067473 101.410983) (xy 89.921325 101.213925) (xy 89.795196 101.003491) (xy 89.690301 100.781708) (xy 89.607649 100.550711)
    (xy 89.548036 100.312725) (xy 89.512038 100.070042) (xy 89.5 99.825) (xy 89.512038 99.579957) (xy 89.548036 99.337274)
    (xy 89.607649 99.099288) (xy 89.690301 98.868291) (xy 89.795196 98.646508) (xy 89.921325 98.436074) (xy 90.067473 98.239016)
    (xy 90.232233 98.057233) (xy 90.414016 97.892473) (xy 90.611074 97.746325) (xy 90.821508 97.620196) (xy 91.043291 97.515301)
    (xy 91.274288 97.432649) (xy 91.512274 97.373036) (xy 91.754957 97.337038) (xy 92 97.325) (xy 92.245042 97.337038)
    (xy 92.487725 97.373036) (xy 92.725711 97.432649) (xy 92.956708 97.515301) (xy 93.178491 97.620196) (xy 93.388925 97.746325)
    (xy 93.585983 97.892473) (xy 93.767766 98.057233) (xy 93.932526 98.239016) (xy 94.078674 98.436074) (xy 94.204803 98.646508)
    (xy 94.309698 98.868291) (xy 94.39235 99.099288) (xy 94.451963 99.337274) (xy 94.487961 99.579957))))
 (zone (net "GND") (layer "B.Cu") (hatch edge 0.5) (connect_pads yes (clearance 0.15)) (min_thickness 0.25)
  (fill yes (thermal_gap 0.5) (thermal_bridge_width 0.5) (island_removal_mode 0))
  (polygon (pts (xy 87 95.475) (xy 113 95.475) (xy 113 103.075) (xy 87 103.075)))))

